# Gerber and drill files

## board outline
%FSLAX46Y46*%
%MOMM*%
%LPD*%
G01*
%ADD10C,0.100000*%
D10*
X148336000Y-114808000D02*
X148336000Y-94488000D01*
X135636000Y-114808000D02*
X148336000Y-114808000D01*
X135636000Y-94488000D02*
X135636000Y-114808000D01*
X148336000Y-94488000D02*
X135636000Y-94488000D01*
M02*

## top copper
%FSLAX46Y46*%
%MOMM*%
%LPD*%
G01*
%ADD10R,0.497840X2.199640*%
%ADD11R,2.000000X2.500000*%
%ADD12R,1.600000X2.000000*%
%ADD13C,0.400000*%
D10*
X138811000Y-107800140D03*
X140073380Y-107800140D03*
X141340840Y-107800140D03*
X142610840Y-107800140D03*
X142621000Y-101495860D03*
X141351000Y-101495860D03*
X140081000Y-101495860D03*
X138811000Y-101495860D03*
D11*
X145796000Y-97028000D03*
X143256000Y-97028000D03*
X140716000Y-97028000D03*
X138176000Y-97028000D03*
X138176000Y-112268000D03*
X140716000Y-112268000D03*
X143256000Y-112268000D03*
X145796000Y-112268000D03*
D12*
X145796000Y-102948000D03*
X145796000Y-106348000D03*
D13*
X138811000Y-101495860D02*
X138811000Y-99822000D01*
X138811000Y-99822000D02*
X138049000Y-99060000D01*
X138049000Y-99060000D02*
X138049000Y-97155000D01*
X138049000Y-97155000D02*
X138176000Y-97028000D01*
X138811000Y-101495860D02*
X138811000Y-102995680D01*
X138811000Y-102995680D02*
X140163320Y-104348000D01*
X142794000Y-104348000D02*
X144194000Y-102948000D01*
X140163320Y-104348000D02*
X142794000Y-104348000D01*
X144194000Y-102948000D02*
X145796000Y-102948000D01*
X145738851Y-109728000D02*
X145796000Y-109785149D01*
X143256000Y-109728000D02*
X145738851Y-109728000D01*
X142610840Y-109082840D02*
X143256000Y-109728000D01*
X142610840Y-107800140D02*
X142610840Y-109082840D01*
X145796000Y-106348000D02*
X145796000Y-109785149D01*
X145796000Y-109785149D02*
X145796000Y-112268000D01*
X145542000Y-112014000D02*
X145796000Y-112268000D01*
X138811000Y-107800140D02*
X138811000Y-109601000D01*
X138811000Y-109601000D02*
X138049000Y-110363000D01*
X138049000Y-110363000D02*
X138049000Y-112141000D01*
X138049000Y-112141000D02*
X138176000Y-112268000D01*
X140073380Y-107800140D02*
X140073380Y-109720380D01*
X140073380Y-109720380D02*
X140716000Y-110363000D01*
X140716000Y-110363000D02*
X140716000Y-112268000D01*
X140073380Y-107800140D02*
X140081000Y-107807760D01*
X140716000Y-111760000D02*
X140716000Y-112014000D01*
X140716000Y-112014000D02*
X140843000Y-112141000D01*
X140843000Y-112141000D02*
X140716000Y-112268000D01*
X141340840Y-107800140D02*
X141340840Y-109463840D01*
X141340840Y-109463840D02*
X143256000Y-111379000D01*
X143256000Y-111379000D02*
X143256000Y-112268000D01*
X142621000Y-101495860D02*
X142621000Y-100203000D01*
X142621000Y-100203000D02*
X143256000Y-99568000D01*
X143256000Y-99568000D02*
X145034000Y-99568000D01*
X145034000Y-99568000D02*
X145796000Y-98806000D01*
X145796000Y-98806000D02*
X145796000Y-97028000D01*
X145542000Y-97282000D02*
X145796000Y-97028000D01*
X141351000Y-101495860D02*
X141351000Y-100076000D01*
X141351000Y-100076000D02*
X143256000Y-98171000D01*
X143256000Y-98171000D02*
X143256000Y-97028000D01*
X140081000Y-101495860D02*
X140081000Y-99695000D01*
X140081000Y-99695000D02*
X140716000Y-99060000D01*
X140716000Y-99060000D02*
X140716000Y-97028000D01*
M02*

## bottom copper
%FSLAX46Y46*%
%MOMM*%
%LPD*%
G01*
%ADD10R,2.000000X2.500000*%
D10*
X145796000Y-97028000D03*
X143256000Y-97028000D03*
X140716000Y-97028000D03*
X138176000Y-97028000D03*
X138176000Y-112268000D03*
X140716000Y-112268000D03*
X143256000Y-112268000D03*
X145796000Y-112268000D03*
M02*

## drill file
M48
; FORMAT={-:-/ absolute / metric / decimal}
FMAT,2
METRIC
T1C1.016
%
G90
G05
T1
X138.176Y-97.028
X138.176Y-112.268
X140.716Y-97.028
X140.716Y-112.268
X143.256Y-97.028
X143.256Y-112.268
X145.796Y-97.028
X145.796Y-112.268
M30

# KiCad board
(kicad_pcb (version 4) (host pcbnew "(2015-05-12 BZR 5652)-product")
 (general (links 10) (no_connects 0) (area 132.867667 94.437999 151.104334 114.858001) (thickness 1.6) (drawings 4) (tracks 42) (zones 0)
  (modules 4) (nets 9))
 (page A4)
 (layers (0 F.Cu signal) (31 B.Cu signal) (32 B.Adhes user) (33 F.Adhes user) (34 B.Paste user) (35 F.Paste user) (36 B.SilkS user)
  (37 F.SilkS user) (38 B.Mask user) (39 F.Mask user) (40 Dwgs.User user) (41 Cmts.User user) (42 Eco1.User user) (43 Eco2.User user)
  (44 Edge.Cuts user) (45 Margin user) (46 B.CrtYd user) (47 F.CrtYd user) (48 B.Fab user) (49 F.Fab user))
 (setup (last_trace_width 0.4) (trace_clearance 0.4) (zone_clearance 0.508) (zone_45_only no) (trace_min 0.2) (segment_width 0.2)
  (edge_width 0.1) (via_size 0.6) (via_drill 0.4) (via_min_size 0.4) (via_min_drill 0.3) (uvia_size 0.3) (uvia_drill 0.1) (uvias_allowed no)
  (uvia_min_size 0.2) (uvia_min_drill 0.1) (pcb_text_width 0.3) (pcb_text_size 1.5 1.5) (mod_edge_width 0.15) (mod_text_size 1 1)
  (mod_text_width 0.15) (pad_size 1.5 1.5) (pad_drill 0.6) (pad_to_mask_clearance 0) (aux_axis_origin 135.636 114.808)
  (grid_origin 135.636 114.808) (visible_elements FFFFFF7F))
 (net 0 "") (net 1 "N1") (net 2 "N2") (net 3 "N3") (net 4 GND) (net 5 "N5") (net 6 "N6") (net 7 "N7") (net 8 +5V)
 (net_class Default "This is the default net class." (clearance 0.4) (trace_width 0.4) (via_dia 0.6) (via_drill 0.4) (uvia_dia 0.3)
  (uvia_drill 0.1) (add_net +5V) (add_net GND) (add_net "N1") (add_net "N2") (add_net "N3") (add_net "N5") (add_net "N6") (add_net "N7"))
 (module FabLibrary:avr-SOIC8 (layer F.Cu) (at 140.716 104.648)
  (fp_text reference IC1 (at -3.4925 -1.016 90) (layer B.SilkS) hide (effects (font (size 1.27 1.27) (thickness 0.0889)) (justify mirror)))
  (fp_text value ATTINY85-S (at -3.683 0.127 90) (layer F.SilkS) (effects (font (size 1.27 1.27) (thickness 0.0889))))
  (pad 1 smd rect (at -1.905 3.15214) (size 0.49784 2.19964) (layers F.Cu F.Paste F.Mask) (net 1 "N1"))
  (pad 2 smd rect (at -0.64262 3.15214) (size 0.49784 2.19964) (layers F.Cu F.Paste F.Mask) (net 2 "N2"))
  (pad 3 smd rect (at 0.62484 3.15214) (size 0.49784 2.19964) (layers F.Cu F.Paste F.Mask) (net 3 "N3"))
  (pad 4 smd rect (at 1.89484 3.15214) (size 0.49784 2.19964) (layers F.Cu F.Paste F.Mask) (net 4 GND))
  (pad 5 smd rect (at 1.905 -3.15214) (size 0.49784 2.19964) (layers F.Cu F.Paste F.Mask) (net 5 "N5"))
  (pad 6 smd rect (at 0.635 -3.15214) (size 0.49784 2.19964) (layers F.Cu F.Paste F.Mask) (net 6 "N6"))
  (pad 7 smd rect (at -0.635 -3.15214) (size 0.49784 2.19964) (layers F.Cu F.Paste F.Mask) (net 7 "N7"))
  (pad 8 smd rect (at -1.905 -3.15214) (size 0.49784 2.19964) (layers F.Cu F.Paste F.Mask) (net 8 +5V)))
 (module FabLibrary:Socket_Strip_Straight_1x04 (layer F.Cu) (at 145.796 97.028 180)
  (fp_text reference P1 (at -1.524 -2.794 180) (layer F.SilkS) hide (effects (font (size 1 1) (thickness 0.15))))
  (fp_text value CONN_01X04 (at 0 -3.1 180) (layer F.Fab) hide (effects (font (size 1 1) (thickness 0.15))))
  (pad 1 thru_hole rect (at 0 0 180) (size 2 2.5) (drill 1.016) (layers *.Mask F.Cu F.SilkS) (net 5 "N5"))
  (pad 2 thru_hole rect (at 2.54 0 180) (size 2 2.5) (drill 1.016) (layers *.Mask F.Cu F.SilkS) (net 6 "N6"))
  (pad 3 thru_hole rect (at 5.08 0 180) (size 2 2.5) (drill 1.016) (layers *.Mask F.Cu F.SilkS) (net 7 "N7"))
  (pad 4 thru_hole rect (at 7.62 0 180) (size 2 2.5) (drill 1.016) (layers *.Mask F.Cu F.SilkS) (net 8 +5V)))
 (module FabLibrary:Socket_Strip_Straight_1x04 (layer F.Cu) (at 138.176 112.268)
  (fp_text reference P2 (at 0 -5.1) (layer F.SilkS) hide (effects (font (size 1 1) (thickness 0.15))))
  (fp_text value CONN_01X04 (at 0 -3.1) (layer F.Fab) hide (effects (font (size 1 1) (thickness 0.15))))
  (pad 1 thru_hole rect (at 0 0) (size 2 2.5) (drill 1.016) (layers *.Mask F.Cu F.SilkS) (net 1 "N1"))
  (pad 2 thru_hole rect (at 2.54 0) (size 2 2.5) (drill 1.016) (layers *.Mask F.Cu F.SilkS) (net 2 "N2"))
  (pad 3 thru_hole rect (at 5.08 0) (size 2 2.5) (drill 1.016) (layers *.Mask F.Cu F.SilkS) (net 3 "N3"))
  (pad 4 thru_hole rect (at 7.62 0) (size 2 2.5) (drill 1.016) (layers *.Mask F.Cu F.SilkS) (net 4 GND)))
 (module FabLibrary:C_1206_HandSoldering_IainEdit (layer F.Cu) (at 145.796 104.648 270)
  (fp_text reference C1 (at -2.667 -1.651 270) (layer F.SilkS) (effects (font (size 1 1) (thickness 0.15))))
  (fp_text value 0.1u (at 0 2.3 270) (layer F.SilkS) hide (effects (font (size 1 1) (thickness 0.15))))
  (pad 1 smd rect (at -1.7 0 270) (size 2 1.6) (layers F.Cu F.Paste F.Mask) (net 8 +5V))
  (pad 2 smd rect (at 1.7 0 270) (size 2 1.6) (layers F.Cu F.Paste F.Mask) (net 4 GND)))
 (gr_line (start 148.336 114.808) (end 148.336 94.488) (angle 90) (layer Edge.Cuts) (width 0.1))
 (gr_line (start 135.636 114.808) (end 148.336 114.808) (angle 90) (layer Edge.Cuts) (width 0.1))
 (gr_line (start 135.636 94.488) (end 135.636 114.808) (angle 90) (layer Edge.Cuts) (width 0.1))
 (gr_line (start 148.336 94.488) (end 135.636 94.488) (angle 90) (layer Edge.Cuts) (width 0.1))
 (segment (start 138.811 101.49586) (end 138.811 99.822) (width 0.4) (layer F.Cu) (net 8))
 (segment (start 138.811 99.822) (end 138.049 99.06) (width 0.4) (layer F.Cu) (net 8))
 (segment (start 138.049 99.06) (end 138.049 97.155) (width 0.4) (layer F.Cu) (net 8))
 (segment (start 138.049 97.155) (end 138.176 97.028) (width 0.4) (layer F.Cu) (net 8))
 (segment (start 138.811 101.49586) (end 138.811 102.99568) (width 0.4) (layer F.Cu) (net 8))
 (segment (start 138.811 102.99568) (end 140.16332 104.348) (width 0.4) (layer F.Cu) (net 8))
 (segment (start 142.794 104.348) (end 144.194 102.948) (width 0.4) (layer F.Cu) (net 8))
 (segment (start 140.16332 104.348) (end 142.794 104.348) (width 0.4) (layer F.Cu) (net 8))
 (segment (start 144.194 102.948) (end 145.796 102.948) (width 0.4) (layer F.Cu) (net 8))
 (segment (start 145.738851 109.728) (end 145.796 109.785149) (width 0.4) (layer F.Cu) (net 4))
 (segment (start 143.256 109.728) (end 145.738851 109.728) (width 0.4) (layer F.Cu) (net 4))
 (segment (start 142.61084 109.08284) (end 143.256 109.728) (width 0.4) (layer F.Cu) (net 4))
 (segment (start 142.61084 107.80014) (end 142.61084 109.08284) (width 0.4) (layer F.Cu) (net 4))
 (segment (start 145.796 106.348) (end 145.796 109.785149) (width 0.4) (layer F.Cu) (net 4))
 (segment (start 145.796 109.785149) (end 145.796 112.268) (width 0.4) (layer F.Cu) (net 4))
 (segment (start 145.542 112.014) (end 145.796 112.268) (width 0.4) (layer F.Cu) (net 4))
 (segment (start 138.811 107.80014) (end 138.811 109.601) (width 0.4) (layer F.Cu) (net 1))
 (segment (start 138.811 109.601) (end 138.049 110.363) (width 0.4) (layer F.Cu) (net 1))
 (segment (start 138.049 110.363) (end 138.049 112.141) (width 0.4) (layer F.Cu) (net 1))
 (segment (start 138.049 112.141) (end 138.176 112.268) (width 0.4) (layer F.Cu) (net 1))
 (segment (start 140.07338 107.80014) (end 140.07338 109.72038) (width 0.4) (layer F.Cu) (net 2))
 (segment (start 140.07338 109.72038) (end 140.716 110.363) (width 0.4) (layer F.Cu) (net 2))
 (segment (start 140.716 110.363) (end 140.716 112.268) (width 0.4) (layer F.Cu) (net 2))
 (segment (start 140.07338 107.80014) (end 140.081 107.80776) (width 0.4) (layer F.Cu) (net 2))
 (segment (start 140.716 111.76) (end 140.716 112.014) (width 0.4) (layer F.Cu) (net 2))
 (segment (start 140.716 112.014) (end 140.843 112.141) (width 0.4) (layer F.Cu) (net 2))
 (segment (start 140.843 112.141) (end 140.716 112.268) (width 0.4) (layer F.Cu) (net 2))
 (segment (start 141.34084 107.80014) (end 141.34084 109.46384) (width 0.4) (layer F.Cu) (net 3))
 (segment (start 141.34084 109.46384) (end 143.256 111.379) (width 0.4) (layer F.Cu) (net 3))
 (segment (start 143.256 111.379) (end 143.256 112.268) (width 0.4) (layer F.Cu) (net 3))
 (segment (start 142.621 101.49586) (end 142.621 100.203) (width 0.4) (layer F.Cu) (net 5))
 (segment (start 142.621 100.203) (end 143.256 99.568) (width 0.4) (layer F.Cu) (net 5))
 (segment (start 143.256 99.568) (end 145.034 99.568) (width 0.4) (layer F.Cu) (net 5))
 (segment (start 145.034 99.568) (end 145.796 98.806) (width 0.4) (layer F.Cu) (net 5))
 (segment (start 145.796 98.806) (end 145.796 97.028) (width 0.4) (layer F.Cu) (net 5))
 (segment (start 145.542 97.282) (end 145.796 97.028) (width 0.4) (layer F.Cu) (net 5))
 (segment (start 141.351 101.49586) (end 141.351 100.076) (width 0.4) (layer F.Cu) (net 6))
 (segment (start 141.351 100.076) (end 143.256 98.171) (width 0.4) (layer F.Cu) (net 6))
 (segment (start 143.256 98.171) (end 143.256 97.028) (width 0.4) (layer F.Cu) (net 6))
 (segment (start 140.081 101.49586) (end 140.081 99.695) (width 0.4) (layer F.Cu) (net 7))
 (segment (start 140.081 99.695) (end 140.716 99.06) (width 0.4) (layer F.Cu) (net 7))
 (segment (start 140.716 99.06) (end 140.716 97.028) (width 0.4) (layer F.Cu) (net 7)))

